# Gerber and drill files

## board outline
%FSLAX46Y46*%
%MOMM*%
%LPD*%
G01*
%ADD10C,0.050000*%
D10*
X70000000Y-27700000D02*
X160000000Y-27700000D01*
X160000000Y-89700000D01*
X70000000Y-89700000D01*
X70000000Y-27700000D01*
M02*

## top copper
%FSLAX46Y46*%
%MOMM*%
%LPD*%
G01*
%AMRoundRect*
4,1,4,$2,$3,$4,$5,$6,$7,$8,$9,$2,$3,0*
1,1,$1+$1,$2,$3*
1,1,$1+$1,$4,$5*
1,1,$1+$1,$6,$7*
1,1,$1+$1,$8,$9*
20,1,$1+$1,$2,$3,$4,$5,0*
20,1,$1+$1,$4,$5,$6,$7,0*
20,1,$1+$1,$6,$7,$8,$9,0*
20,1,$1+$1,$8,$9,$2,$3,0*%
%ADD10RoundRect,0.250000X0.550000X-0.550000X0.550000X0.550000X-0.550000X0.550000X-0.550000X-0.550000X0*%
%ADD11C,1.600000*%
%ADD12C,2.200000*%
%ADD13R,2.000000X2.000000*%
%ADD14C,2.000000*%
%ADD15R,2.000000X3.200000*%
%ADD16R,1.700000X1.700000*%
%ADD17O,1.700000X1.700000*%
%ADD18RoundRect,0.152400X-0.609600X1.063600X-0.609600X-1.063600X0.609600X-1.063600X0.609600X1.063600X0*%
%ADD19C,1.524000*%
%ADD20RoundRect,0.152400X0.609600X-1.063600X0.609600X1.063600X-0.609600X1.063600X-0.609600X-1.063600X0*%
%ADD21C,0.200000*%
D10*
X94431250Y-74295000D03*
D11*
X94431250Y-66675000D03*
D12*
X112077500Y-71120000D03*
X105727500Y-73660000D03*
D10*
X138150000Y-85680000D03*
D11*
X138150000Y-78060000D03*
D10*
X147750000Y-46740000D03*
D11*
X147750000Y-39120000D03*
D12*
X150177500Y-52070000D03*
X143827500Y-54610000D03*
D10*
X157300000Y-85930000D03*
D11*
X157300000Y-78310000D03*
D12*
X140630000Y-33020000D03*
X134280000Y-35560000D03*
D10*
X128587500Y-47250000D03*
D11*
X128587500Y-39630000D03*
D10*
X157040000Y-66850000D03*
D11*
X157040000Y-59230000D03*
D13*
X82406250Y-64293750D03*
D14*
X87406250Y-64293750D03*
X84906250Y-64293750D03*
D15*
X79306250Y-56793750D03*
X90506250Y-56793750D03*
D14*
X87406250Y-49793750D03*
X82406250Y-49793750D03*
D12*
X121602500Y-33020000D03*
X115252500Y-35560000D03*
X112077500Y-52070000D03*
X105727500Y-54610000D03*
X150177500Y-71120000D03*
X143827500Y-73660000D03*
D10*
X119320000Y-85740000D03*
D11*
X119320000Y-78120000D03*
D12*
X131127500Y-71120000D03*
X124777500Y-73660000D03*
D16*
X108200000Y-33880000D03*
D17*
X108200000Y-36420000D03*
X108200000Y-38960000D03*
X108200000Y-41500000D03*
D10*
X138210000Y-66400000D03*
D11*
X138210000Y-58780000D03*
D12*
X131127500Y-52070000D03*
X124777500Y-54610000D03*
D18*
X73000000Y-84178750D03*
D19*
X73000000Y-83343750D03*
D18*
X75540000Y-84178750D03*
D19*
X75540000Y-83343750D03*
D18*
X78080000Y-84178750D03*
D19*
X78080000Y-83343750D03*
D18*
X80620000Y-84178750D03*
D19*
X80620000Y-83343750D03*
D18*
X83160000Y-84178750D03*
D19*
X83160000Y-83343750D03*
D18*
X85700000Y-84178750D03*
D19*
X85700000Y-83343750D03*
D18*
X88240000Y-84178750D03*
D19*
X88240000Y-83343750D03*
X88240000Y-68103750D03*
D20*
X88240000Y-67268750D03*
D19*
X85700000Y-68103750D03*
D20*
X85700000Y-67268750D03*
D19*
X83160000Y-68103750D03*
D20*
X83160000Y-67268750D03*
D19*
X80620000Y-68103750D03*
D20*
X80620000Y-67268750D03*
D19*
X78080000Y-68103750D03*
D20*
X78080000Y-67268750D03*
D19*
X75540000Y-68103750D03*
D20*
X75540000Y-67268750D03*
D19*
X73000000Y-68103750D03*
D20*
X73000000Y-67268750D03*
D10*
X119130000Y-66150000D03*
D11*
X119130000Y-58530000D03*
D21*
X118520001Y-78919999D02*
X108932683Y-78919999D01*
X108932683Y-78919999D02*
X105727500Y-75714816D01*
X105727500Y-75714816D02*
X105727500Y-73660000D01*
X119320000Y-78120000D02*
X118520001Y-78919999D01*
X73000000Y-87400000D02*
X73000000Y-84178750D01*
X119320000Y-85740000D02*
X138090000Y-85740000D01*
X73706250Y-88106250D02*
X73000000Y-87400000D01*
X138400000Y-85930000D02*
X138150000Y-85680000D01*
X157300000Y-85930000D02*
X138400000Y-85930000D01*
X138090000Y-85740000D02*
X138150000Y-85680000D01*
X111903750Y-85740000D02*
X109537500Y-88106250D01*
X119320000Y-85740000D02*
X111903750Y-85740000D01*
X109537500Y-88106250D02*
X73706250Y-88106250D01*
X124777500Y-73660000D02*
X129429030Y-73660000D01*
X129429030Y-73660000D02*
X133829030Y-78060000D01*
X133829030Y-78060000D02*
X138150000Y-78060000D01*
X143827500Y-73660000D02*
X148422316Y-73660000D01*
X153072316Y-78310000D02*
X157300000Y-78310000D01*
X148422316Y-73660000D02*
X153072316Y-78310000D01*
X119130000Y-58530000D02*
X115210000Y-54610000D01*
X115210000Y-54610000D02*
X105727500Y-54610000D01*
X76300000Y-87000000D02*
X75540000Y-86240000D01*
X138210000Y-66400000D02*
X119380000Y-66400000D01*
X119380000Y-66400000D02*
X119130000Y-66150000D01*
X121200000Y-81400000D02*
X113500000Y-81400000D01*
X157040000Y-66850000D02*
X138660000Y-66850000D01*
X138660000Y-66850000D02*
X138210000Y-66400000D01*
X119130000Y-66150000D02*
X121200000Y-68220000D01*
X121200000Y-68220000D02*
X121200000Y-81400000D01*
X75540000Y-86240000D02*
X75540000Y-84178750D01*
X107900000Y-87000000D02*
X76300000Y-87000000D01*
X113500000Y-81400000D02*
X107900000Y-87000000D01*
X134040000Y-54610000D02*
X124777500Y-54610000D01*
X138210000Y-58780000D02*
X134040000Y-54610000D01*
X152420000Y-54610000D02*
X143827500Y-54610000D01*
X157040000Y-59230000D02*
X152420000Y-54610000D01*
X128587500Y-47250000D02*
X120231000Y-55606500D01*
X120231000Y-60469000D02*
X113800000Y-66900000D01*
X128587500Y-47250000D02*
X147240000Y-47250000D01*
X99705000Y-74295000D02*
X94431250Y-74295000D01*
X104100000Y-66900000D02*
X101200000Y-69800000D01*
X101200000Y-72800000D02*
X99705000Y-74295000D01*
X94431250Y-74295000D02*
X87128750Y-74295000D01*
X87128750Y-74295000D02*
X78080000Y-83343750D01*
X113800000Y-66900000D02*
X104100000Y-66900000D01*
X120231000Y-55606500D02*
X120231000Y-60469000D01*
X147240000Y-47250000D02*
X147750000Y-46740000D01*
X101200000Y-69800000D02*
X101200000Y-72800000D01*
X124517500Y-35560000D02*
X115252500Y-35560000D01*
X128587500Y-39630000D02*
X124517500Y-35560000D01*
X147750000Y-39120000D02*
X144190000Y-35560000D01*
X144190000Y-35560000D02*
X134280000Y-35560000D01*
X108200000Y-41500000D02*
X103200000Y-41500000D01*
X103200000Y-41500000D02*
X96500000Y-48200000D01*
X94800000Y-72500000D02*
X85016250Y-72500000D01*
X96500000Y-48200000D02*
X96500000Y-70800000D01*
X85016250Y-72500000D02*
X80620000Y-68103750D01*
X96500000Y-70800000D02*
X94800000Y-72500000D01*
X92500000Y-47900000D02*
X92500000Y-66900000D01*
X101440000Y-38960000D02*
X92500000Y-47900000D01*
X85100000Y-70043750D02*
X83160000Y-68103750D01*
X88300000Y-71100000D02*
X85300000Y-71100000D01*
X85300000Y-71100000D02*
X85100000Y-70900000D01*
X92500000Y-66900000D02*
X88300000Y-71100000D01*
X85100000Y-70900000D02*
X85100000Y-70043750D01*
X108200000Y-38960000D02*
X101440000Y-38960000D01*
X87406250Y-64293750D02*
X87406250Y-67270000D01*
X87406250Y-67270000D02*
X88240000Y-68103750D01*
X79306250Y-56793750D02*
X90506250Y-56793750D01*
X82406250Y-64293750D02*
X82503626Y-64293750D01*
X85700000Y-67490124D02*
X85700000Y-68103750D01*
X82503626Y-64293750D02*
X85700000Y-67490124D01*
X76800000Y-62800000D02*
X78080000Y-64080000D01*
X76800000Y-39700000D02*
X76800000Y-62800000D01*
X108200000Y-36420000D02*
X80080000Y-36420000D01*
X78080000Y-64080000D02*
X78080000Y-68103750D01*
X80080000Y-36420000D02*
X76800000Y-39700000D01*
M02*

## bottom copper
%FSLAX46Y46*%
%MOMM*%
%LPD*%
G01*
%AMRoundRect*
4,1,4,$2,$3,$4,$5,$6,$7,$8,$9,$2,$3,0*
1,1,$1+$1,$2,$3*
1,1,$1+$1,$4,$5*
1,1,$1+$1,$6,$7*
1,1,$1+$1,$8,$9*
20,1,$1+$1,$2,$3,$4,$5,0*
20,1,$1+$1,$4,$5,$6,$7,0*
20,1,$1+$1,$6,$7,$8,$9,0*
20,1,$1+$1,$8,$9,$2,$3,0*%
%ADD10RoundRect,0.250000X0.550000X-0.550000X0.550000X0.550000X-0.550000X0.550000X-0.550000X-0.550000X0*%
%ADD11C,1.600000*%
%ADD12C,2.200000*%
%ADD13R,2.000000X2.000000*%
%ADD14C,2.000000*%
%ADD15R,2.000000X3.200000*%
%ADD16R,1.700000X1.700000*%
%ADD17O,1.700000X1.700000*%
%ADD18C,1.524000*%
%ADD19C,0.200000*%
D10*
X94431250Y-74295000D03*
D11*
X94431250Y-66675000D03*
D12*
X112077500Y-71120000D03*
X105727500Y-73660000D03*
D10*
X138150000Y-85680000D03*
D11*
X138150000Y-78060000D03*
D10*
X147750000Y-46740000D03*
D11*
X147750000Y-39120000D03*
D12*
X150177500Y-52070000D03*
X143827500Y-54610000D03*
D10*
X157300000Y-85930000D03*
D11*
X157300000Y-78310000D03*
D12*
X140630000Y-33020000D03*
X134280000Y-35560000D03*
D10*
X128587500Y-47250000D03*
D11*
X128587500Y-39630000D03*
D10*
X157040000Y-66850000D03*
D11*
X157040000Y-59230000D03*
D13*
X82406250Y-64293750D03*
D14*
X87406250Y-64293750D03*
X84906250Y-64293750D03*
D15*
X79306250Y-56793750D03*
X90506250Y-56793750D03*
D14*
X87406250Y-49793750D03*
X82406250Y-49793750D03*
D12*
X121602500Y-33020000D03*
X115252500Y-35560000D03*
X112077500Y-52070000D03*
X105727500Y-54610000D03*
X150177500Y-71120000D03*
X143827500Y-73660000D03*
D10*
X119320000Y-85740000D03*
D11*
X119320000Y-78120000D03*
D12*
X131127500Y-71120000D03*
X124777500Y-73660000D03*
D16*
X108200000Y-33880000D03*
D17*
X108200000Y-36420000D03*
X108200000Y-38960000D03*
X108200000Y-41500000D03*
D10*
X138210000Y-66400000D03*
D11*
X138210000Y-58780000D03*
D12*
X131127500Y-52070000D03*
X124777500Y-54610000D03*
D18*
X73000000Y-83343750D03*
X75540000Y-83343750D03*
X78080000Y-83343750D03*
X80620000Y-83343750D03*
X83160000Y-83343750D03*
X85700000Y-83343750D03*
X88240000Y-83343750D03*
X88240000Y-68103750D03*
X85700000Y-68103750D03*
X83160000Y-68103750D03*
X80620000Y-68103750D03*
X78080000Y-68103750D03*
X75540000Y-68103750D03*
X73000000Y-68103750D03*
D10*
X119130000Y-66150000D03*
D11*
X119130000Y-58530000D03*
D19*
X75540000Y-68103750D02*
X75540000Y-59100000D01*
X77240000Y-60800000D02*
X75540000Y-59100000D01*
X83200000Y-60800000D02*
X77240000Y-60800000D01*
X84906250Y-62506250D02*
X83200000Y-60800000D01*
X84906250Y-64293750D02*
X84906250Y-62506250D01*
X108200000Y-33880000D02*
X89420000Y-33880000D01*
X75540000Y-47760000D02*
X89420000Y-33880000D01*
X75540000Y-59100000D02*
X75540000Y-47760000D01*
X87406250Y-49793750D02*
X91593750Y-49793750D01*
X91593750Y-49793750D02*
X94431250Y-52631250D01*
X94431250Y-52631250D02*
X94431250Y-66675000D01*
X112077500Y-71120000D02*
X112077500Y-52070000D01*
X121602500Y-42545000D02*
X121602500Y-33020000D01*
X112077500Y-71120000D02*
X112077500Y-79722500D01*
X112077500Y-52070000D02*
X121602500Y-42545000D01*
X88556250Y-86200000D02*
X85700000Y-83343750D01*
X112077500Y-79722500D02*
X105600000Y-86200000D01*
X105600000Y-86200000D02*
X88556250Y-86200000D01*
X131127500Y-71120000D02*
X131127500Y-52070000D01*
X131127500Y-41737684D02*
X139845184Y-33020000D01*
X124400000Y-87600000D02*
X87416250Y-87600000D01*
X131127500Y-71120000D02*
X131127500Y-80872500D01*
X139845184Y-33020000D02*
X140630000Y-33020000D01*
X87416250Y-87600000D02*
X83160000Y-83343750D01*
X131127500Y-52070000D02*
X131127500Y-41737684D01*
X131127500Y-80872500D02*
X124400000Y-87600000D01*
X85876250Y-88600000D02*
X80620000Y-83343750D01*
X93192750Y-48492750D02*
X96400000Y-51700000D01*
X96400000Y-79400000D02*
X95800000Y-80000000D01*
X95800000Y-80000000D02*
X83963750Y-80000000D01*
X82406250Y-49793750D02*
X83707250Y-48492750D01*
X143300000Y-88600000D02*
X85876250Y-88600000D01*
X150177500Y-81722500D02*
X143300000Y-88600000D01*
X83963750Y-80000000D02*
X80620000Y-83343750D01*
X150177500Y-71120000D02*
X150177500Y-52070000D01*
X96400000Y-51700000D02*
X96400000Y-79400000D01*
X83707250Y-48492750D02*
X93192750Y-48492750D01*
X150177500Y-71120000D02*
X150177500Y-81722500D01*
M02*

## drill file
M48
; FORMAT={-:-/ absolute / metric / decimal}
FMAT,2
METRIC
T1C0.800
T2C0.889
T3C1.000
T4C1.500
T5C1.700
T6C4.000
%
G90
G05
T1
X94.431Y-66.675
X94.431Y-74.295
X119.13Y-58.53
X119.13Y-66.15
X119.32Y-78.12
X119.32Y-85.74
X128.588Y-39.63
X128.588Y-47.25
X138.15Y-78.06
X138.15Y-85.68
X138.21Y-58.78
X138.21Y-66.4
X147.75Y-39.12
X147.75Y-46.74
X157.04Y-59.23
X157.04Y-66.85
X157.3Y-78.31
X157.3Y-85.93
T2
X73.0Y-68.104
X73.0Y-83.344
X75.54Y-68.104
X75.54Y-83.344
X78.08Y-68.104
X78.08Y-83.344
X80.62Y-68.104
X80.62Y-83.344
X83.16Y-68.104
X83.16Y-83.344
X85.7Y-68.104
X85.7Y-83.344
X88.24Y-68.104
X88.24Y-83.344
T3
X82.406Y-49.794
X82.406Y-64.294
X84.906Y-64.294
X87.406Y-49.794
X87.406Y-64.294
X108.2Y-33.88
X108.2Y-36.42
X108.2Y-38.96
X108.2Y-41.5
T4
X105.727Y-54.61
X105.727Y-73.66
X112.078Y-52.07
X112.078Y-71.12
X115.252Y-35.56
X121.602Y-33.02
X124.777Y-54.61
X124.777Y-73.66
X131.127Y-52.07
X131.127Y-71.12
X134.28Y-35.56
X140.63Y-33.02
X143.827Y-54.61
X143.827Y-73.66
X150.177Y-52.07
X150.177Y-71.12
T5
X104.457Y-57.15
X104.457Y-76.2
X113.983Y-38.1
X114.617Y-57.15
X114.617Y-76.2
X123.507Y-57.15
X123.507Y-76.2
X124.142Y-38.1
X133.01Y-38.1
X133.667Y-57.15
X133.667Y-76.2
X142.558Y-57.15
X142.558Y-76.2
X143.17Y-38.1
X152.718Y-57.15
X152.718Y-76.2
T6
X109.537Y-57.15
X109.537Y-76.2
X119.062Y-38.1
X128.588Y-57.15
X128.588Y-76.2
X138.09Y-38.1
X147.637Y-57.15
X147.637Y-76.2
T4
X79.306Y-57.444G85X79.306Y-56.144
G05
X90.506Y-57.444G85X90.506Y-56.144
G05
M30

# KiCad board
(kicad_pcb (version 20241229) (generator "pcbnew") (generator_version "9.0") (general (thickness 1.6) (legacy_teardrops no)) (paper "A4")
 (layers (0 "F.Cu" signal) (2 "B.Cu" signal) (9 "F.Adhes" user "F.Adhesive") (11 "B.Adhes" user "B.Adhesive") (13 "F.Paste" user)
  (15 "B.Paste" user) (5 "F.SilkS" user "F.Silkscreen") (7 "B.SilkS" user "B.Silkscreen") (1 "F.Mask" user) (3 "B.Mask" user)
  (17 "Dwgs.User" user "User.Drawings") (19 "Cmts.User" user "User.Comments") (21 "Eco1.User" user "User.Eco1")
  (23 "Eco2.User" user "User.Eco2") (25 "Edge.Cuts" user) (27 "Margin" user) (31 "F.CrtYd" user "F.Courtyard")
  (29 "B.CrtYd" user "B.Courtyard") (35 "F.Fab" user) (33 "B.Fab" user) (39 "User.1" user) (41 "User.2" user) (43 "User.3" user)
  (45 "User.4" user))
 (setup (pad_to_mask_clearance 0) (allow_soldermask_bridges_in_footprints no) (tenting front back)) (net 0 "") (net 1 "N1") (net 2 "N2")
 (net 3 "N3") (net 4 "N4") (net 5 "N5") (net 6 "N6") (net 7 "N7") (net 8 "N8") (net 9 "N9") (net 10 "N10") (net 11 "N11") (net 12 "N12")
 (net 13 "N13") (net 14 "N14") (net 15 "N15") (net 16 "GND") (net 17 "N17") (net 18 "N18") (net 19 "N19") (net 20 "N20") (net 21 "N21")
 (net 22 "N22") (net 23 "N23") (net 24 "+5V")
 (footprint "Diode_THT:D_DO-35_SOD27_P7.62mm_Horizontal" (layer "F.Cu") (at 94.43125 74.295 90)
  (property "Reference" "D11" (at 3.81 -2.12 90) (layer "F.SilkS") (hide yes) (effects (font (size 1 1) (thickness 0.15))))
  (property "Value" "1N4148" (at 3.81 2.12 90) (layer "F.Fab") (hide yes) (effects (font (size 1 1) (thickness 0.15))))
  (pad "1" thru_hole roundrect (at 0 0 90) (size 1.6 1.6) (drill 0.8) (layers "*.Cu" "*.Mask") (remove_unused_layers no)
   (roundrect_rratio 0.15625) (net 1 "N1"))
  (pad "2" thru_hole circle (at 7.62 0 90) (size 1.6 1.6) (drill 0.8) (layers "*.Cu" "*.Mask") (remove_unused_layers no) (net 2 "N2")))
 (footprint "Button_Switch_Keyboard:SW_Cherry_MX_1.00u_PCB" (layer "F.Cu") (at 112.0775 71.12)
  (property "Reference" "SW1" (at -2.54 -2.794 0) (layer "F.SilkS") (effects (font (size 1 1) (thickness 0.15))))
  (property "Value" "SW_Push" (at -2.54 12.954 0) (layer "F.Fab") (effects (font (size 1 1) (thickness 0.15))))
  (pad "" np_thru_hole circle (at -7.62 5.08) (size 1.7 1.7) (drill 1.7) (layers "*.Cu" "*.Mask"))
  (pad "" np_thru_hole circle (at -2.54 5.08) (size 4 4) (drill 4) (layers "*.Cu" "*.Mask"))
  (pad "" np_thru_hole circle (at 2.54 5.08) (size 1.7 1.7) (drill 1.7) (layers "*.Cu" "*.Mask"))
  (pad "1" thru_hole circle (at 0 0) (size 2.2 2.2) (drill 1.5) (layers "*.Cu" "*.Mask") (remove_unused_layers no) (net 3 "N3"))
  (pad "2" thru_hole circle (at -6.35 2.54) (size 2.2 2.2) (drill 1.5) (layers "*.Cu" "*.Mask") (remove_unused_layers no) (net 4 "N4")))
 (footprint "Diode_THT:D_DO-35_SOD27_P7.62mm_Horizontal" (layer "F.Cu") (at 138.15 85.68 90)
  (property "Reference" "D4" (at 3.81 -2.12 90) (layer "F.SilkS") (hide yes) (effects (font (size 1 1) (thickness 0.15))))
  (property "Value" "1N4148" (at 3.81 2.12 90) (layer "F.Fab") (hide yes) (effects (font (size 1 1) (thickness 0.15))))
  (pad "1" thru_hole roundrect (at 0 0 90) (size 1.6 1.6) (drill 0.8) (layers "*.Cu" "*.Mask") (remove_unused_layers no)
   (roundrect_rratio 0.15625) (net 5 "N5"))
  (pad "2" thru_hole circle (at 7.62 0 90) (size 1.6 1.6) (drill 0.8) (layers "*.Cu" "*.Mask") (remove_unused_layers no) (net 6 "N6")))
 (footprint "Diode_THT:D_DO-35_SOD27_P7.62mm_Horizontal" (layer "F.Cu") (at 147.75 46.74 90)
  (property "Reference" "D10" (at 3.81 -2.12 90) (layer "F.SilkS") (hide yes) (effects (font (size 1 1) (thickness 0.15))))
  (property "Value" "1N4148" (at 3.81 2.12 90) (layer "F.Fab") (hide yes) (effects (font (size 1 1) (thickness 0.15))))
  (pad "1" thru_hole roundrect (at 0 0 90) (size 1.6 1.6) (drill 0.8) (layers "*.Cu" "*.Mask") (remove_unused_layers no)
   (roundrect_rratio 0.15625) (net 1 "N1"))
  (pad "2" thru_hole circle (at 7.62 0 90) (size 1.6 1.6) (drill 0.8) (layers "*.Cu" "*.Mask") (remove_unused_layers no) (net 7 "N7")))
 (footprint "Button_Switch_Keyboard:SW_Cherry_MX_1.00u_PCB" (layer "F.Cu") (at 150.1775 52.07)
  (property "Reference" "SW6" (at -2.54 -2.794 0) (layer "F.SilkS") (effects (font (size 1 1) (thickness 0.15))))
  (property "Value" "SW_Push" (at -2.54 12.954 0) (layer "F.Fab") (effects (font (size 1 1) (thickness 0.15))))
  (pad "" np_thru_hole circle (at -7.62 5.08) (size 1.7 1.7) (drill 1.7) (layers "*.Cu" "*.Mask"))
  (pad "" np_thru_hole circle (at -2.54 5.08) (size 4 4) (drill 4) (layers "*.Cu" "*.Mask"))
  (pad "" np_thru_hole circle (at 2.54 5.08) (size 1.7 1.7) (drill 1.7) (layers "*.Cu" "*.Mask"))
  (pad "1" thru_hole circle (at 0 0) (size 2.2 2.2) (drill 1.5) (layers "*.Cu" "*.Mask") (remove_unused_layers no) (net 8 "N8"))
  (pad "2" thru_hole circle (at -6.35 2.54) (size 2.2 2.2) (drill 1.5) (layers "*.Cu" "*.Mask") (remove_unused_layers no) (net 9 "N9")))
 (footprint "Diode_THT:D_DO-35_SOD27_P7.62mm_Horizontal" (layer "F.Cu") (at 157.3 85.93 90)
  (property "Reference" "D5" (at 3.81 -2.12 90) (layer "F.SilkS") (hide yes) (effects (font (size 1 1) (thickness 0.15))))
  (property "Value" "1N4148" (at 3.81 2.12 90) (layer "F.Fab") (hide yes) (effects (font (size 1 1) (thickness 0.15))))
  (pad "1" thru_hole roundrect (at 0 0 90) (size 1.6 1.6) (drill 0.8) (layers "*.Cu" "*.Mask") (remove_unused_layers no)
   (roundrect_rratio 0.15625) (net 5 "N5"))
  (pad "2" thru_hole circle (at 7.62 0 90) (size 1.6 1.6) (drill 0.8) (layers "*.Cu" "*.Mask") (remove_unused_layers no) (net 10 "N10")))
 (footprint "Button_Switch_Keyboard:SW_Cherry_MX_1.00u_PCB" (layer "F.Cu") (at 140.63 33.02)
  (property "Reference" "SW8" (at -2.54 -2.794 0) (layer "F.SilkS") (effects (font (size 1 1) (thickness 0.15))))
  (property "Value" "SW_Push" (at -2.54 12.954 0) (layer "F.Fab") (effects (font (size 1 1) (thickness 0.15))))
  (pad "" np_thru_hole circle (at -7.62 5.08) (size 1.7 1.7) (drill 1.7) (layers "*.Cu" "*.Mask"))
  (pad "" np_thru_hole circle (at -2.54 5.08) (size 4 4) (drill 4) (layers "*.Cu" "*.Mask"))
  (pad "" np_thru_hole circle (at 2.54 5.08) (size 1.7 1.7) (drill 1.7) (layers "*.Cu" "*.Mask"))
  (pad "1" thru_hole circle (at 0 0) (size 2.2 2.2) (drill 1.5) (layers "*.Cu" "*.Mask") (remove_unused_layers no) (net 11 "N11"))
  (pad "2" thru_hole circle (at -6.35 2.54) (size 2.2 2.2) (drill 1.5) (layers "*.Cu" "*.Mask") (remove_unused_layers no) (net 7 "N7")))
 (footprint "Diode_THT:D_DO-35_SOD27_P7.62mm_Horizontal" (layer "F.Cu") (at 128.5875 47.25 90)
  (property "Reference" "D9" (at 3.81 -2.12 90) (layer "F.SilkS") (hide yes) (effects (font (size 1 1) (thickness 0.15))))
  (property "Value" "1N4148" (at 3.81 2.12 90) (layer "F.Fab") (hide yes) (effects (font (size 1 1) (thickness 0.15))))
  (pad "1" thru_hole roundrect (at 0 0 90) (size 1.6 1.6) (drill 0.8) (layers "*.Cu" "*.Mask") (remove_unused_layers no)
   (roundrect_rratio 0.15625) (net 1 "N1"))
  (pad "2" thru_hole circle (at 7.62 0 90) (size 1.6 1.6) (drill 0.8) (layers "*.Cu" "*.Mask") (remove_unused_layers no) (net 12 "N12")))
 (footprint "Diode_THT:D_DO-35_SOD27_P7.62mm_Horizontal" (layer "F.Cu") (at 157.04 66.85 90)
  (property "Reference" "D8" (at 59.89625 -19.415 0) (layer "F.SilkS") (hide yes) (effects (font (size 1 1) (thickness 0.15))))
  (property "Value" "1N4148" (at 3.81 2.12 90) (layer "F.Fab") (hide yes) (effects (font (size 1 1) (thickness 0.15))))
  (pad "1" thru_hole roundrect (at 0 0 90) (size 1.6 1.6) (drill 0.8) (layers "*.Cu" "*.Mask") (remove_unused_layers no)
   (roundrect_rratio 0.15625) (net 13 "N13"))
  (pad "2" thru_hole circle (at 7.62 0 90) (size 1.6 1.6) (drill 0.8) (layers "*.Cu" "*.Mask") (remove_unused_layers no) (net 9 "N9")))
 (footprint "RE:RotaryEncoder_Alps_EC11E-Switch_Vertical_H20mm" (layer "F.Cu") (at 82.40625 64.29375 90)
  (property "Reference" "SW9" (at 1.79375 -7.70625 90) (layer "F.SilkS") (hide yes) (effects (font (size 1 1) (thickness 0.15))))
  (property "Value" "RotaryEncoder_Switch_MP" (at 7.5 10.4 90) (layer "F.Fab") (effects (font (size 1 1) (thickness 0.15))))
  (pad "A" thru_hole rect (at 0 0 90) (size 2 2) (drill 1) (layers "*.Cu" "*.Mask") (remove_unused_layers no) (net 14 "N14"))
  (pad "B" thru_hole circle (at 0 5 90) (size 2 2) (drill 1) (layers "*.Cu" "*.Mask") (remove_unused_layers no) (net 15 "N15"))
  (pad "C" thru_hole circle (at 0 2.5 90) (size 2 2) (drill 1) (layers "*.Cu" "*.Mask") (remove_unused_layers no) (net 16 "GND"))
  (pad "MP" thru_hole rect (at 7.5 -3.1 90) (size 3.2 2) (drill oval 2.8 1.5) (layers "*.Cu" "*.Mask") (remove_unused_layers no)
   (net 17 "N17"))
  (pad "MP" thru_hole rect (at 7.5 8.1 90) (size 3.2 2) (drill oval 2.8 1.5) (layers "*.Cu" "*.Mask") (remove_unused_layers no)
   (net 17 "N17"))
  (pad "S1" thru_hole circle (at 14.5 5 90) (size 2 2) (drill 1) (layers "*.Cu" "*.Mask") (remove_unused_layers no) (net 2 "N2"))
  (pad "S2" thru_hole circle (at 14.5 0 90) (size 2 2) (drill 1) (layers "*.Cu" "*.Mask") (remove_unused_layers no) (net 8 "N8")))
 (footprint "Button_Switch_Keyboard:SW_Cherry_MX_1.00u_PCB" (layer "F.Cu") (at 121.6025 33.02)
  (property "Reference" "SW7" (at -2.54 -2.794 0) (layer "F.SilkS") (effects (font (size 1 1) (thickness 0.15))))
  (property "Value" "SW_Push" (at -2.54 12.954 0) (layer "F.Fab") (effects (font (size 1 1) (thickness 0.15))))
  (pad "" np_thru_hole circle (at -7.62 5.08) (size 1.7 1.7) (drill 1.7) (layers "*.Cu" "*.Mask"))
  (pad "" np_thru_hole circle (at -2.54 5.08) (size 4 4) (drill 4) (layers "*.Cu" "*.Mask"))
  (pad "" np_thru_hole circle (at 2.54 5.08) (size 1.7 1.7) (drill 1.7) (layers "*.Cu" "*.Mask"))
  (pad "1" thru_hole circle (at 0 0) (size 2.2 2.2) (drill 1.5) (layers "*.Cu" "*.Mask") (remove_unused_layers no) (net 3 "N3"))
  (pad "2" thru_hole circle (at -6.35 2.54) (size 2.2 2.2) (drill 1.5) (layers "*.Cu" "*.Mask") (remove_unused_layers no) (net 12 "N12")))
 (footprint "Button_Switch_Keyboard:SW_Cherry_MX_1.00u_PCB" (layer "F.Cu") (at 112.0775 52.07)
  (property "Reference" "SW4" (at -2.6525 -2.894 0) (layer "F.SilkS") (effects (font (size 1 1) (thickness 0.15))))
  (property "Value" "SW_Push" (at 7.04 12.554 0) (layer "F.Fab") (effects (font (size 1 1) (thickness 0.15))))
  (pad "" np_thru_hole circle (at -7.62 5.08) (size 1.7 1.7) (drill 1.7) (layers "*.Cu" "*.Mask"))
  (pad "" np_thru_hole circle (at -2.54 5.08) (size 4 4) (drill 4) (layers "*.Cu" "*.Mask"))
  (pad "" np_thru_hole circle (at 2.54 5.08) (size 1.7 1.7) (drill 1.7) (layers "*.Cu" "*.Mask"))
  (pad "1" thru_hole circle (at 0 0) (size 2.2 2.2) (drill 1.5) (layers "*.Cu" "*.Mask") (remove_unused_layers no) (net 3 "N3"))
  (pad "2" thru_hole circle (at -6.35 2.54) (size 2.2 2.2) (drill 1.5) (layers "*.Cu" "*.Mask") (remove_unused_layers no) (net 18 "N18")))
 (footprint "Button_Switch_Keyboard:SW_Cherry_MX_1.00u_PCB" (layer "F.Cu") (at 150.1775 71.12)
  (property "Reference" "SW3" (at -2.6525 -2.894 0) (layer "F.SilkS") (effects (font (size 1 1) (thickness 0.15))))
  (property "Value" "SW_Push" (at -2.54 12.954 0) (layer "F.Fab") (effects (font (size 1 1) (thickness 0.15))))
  (pad "" np_thru_hole circle (at -7.62 5.08) (size 1.7 1.7) (drill 1.7) (layers "*.Cu" "*.Mask"))
  (pad "" np_thru_hole circle (at -2.54 5.08) (size 4 4) (drill 4) (layers "*.Cu" "*.Mask"))
  (pad "" np_thru_hole circle (at 2.54 5.08) (size 1.7 1.7) (drill 1.7) (layers "*.Cu" "*.Mask"))
  (pad "1" thru_hole circle (at 0 0) (size 2.2 2.2) (drill 1.5) (layers "*.Cu" "*.Mask") (remove_unused_layers no) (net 8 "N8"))
  (pad "2" thru_hole circle (at -6.35 2.54) (size 2.2 2.2) (drill 1.5) (layers "*.Cu" "*.Mask") (remove_unused_layers no) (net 10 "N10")))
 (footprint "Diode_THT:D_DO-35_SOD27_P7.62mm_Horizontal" (layer "F.Cu") (at 119.32 85.74 90)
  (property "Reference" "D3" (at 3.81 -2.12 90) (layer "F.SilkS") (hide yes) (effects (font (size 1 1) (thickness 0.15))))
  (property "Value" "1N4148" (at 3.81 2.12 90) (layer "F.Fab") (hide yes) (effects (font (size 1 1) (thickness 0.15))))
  (pad "1" thru_hole roundrect (at 0 0 90) (size 1.6 1.6) (drill 0.8) (layers "*.Cu" "*.Mask") (remove_unused_layers no)
   (roundrect_rratio 0.15625) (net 5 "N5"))
  (pad "2" thru_hole circle (at 7.62 0 90) (size 1.6 1.6) (drill 0.8) (layers "*.Cu" "*.Mask") (remove_unused_layers no) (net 4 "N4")))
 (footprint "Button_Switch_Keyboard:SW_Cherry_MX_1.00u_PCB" (layer "F.Cu") (at 131.1275 71.12)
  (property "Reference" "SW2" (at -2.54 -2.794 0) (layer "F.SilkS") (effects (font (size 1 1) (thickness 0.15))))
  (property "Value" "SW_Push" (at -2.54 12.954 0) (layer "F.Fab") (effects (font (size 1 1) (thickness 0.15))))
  (pad "" np_thru_hole circle (at -7.62 5.08) (size 1.7 1.7) (drill 1.7) (layers "*.Cu" "*.Mask"))
  (pad "" np_thru_hole circle (at -2.54 5.08) (size 4 4) (drill 4) (layers "*.Cu" "*.Mask"))
  (pad "" np_thru_hole circle (at 2.54 5.08) (size 1.7 1.7) (drill 1.7) (layers "*.Cu" "*.Mask"))
  (pad "1" thru_hole circle (at 0 0) (size 2.2 2.2) (drill 1.5) (layers "*.Cu" "*.Mask") (remove_unused_layers no) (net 11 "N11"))
  (pad "2" thru_hole circle (at -6.35 2.54) (size 2.2 2.2) (drill 1.5) (layers "*.Cu" "*.Mask") (remove_unused_layers no) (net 6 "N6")))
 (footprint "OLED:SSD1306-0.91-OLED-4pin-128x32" (layer "F.Cu") (at 71.7 31.69)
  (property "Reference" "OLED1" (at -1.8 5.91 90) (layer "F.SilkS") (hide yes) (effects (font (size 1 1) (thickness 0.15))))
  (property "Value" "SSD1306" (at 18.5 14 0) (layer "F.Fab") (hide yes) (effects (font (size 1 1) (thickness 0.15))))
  (pad "1" thru_hole rect (at 36.5 2.19) (size 1.7 1.7) (drill 1) (layers "*.Cu" "*.Mask") (remove_unused_layers no) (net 16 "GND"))
  (pad "2" thru_hole oval (at 36.5 4.73) (size 1.7 1.7) (drill 1) (layers "*.Cu" "*.Mask") (remove_unused_layers no) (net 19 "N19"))
  (pad "3" thru_hole oval (at 36.5 7.27) (size 1.7 1.7) (drill 1) (layers "*.Cu" "*.Mask") (remove_unused_layers no) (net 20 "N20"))
  (pad "4" thru_hole oval (at 36.5 9.81) (size 1.7 1.7) (drill 1) (layers "*.Cu" "*.Mask") (remove_unused_layers no) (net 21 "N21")))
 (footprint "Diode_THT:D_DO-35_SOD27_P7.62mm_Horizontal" (layer "F.Cu") (at 138.21 66.4 90)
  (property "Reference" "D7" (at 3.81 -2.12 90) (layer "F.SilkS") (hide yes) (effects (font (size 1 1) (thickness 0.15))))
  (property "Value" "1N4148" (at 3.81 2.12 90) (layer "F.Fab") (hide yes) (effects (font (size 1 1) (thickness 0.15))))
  (pad "1" thru_hole roundrect (at 0 0 90) (size 1.6 1.6) (drill 0.8) (layers "*.Cu" "*.Mask") (remove_unused_layers no)
   (roundrect_rratio 0.15625) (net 13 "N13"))
  (pad "2" thru_hole circle (at 7.62 0 90) (size 1.6 1.6) (drill 0.8) (layers "*.Cu" "*.Mask") (remove_unused_layers no) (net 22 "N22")))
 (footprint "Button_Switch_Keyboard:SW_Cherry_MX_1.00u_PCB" (layer "F.Cu") (at 131.1275 52.07)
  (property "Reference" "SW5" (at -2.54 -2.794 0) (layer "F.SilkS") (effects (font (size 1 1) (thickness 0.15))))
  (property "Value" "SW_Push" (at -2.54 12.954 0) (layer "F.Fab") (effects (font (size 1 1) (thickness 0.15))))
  (pad "" np_thru_hole circle (at -7.62 5.08) (size 1.7 1.7) (drill 1.7) (layers "*.Cu" "*.Mask"))
  (pad "" np_thru_hole circle (at -2.54 5.08) (size 4 4) (drill 4) (layers "*.Cu" "*.Mask"))
  (pad "" np_thru_hole circle (at 2.54 5.08) (size 1.7 1.7) (drill 1.7) (layers "*.Cu" "*.Mask"))
  (pad "1" thru_hole circle (at 0 0) (size 2.2 2.2) (drill 1.5) (layers "*.Cu" "*.Mask") (remove_unused_layers no) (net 11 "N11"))
  (pad "2" thru_hole circle (at -6.35 2.54) (size 2.2 2.2) (drill 1.5) (layers "*.Cu" "*.Mask") (remove_unused_layers no) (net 22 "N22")))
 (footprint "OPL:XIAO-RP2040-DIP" (layer "F.Cu") (at 80.62 75.72375 90)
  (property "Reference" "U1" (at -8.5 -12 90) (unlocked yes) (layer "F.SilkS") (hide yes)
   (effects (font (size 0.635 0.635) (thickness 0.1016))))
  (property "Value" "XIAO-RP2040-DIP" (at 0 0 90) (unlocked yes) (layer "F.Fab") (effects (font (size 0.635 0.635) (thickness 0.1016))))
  (pad "1" smd roundrect (at -8.455 -7.62 270) (size 2.432 1.524) (layers "F.Cu" "F.Mask") (roundrect_rratio 0.1) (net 5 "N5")
   (thermal_bridge_angle 45))
  (pad "1" thru_hole circle (at -7.62 -7.62 270) (size 1.524 1.524) (drill 0.889) (layers "*.Cu" "*.Mask") (remove_unused_layers no)
   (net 5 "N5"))
  (pad "2" smd roundrect (at -8.455 -5.08 270) (size 2.432 1.524) (layers "F.Cu" "F.Mask") (roundrect_rratio 0.1) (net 13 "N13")
   (thermal_bridge_angle 45))
  (pad "2" thru_hole circle (at -7.62 -5.08 270) (size 1.524 1.524) (drill 0.889) (layers "*.Cu" "*.Mask") (remove_unused_layers no)
   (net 13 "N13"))
  (pad "3" smd roundrect (at -8.455 -2.54 270) (size 2.432 1.524) (layers "F.Cu" "F.Mask") (roundrect_rratio 0.1) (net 1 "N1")
   (thermal_bridge_angle 45))
  (pad "3" thru_hole circle (at -7.62 -2.54 270) (size 1.524 1.524) (drill 0.889) (layers "*.Cu" "*.Mask") (remove_unused_layers no)
   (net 1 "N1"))
  (pad "4" smd roundrect (at -8.455 0 270) (size 2.432 1.524) (layers "F.Cu" "F.Mask") (roundrect_rratio 0.1) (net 8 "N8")
   (thermal_bridge_angle 45))
  (pad "4" thru_hole circle (at -7.62 0 270) (size 1.524 1.524) (drill 0.889) (layers "*.Cu" "*.Mask") (remove_unused_layers no)
   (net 8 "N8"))
  (pad "5" smd roundrect (at -8.455 2.54 270) (size 2.432 1.524) (layers "F.Cu" "F.Mask") (roundrect_rratio 0.1) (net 11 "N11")
   (thermal_bridge_angle 45))
  (pad "5" thru_hole circle (at -7.62 2.54 270) (size 1.524 1.524) (drill 0.889) (layers "*.Cu" "*.Mask") (remove_unused_layers no)
   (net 11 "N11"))
  (pad "6" smd roundrect (at -8.455 5.08 270) (size 2.432 1.524) (layers "F.Cu" "F.Mask") (roundrect_rratio 0.1) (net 3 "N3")
   (thermal_bridge_angle 45))
  (pad "6" thru_hole circle (at -7.62 5.08 270) (size 1.524 1.524) (drill 0.889) (layers "*.Cu" "*.Mask") (remove_unused_layers no)
   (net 3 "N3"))
  (pad "7" smd roundrect (at -8.455 7.62 270) (size 2.432 1.524) (layers "F.Cu" "F.Mask") (roundrect_rratio 0.1) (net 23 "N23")
   (thermal_bridge_angle 45))
  (pad "7" thru_hole circle (at -7.62 7.62 270) (size 1.524 1.524) (drill 0.889) (layers "*.Cu" "*.Mask") (remove_unused_layers no)
   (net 23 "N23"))
  (pad "8" thru_hole circle (at 7.62 7.62 90) (size 1.524 1.524) (drill 0.889) (layers "*.Cu" "*.Mask") (remove_unused_layers no)
   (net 15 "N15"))
  (pad "8" smd roundrect (at 8.455 7.62 90) (size 2.432 1.524) (layers "F.Cu" "F.Mask") (roundrect_rratio 0.1) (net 15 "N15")
   (thermal_bridge_angle 45))
  (pad "9" thru_hole circle (at 7.62 5.08 90) (size 1.524 1.524) (drill 0.889) (layers "*.Cu" "*.Mask") (remove_unused_layers no)
   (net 14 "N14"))
  (pad "9" smd roundrect (at 8.455 5.08 90) (size 2.432 1.524) (layers "F.Cu" "F.Mask") (roundrect_rratio 0.1) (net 14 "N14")
   (thermal_bridge_angle 45))
  (pad "10" thru_hole circle (at 7.62 2.54 90) (size 1.524 1.524) (drill 0.889) (layers "*.Cu" "*.Mask") (remove_unused_layers no)
   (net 20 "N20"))
  (pad "10" smd roundrect (at 8.455 2.54 90) (size 2.432 1.524) (layers "F.Cu" "F.Mask") (roundrect_rratio 0.1) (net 20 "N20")
   (thermal_bridge_angle 45))
  (pad "11" thru_hole circle (at 7.62 0 90) (size 1.524 1.524) (drill 0.889) (layers "*.Cu" "*.Mask") (remove_unused_layers no)
   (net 21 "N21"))
  (pad "11" smd roundrect (at 8.455 0 90) (size 2.432 1.524) (layers "F.Cu" "F.Mask") (roundrect_rratio 0.1) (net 21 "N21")
   (thermal_bridge_angle 45))
  (pad "12" thru_hole circle (at 7.62 -2.54 90) (size 1.524 1.524) (drill 0.889) (layers "*.Cu" "*.Mask") (remove_unused_layers no)
   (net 19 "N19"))
  (pad "12" smd roundrect (at 8.455 -2.54 90) (size 2.432 1.524) (layers "F.Cu" "F.Mask") (roundrect_rratio 0.1) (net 19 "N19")
   (thermal_bridge_angle 45))
  (pad "13" thru_hole circle (at 7.62 -5.08 90) (size 1.524 1.524) (drill 0.889) (layers "*.Cu" "*.Mask") (remove_unused_layers no)
   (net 16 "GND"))
  (pad "13" smd roundrect (at 8.455 -5.08 90) (size 2.432 1.524) (layers "F.Cu" "F.Mask") (roundrect_rratio 0.1) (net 16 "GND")
   (thermal_bridge_angle 45))
  (pad "14" thru_hole circle (at 7.62 -7.62 90) (size 1.524 1.524) (drill 0.889) (layers "*.Cu" "*.Mask") (remove_unused_layers no)
   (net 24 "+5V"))
  (pad "14" smd roundrect (at 8.455 -7.62 90) (size 2.432 1.524) (layers "F.Cu" "F.Mask") (roundrect_rratio 0.1) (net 24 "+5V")
   (thermal_bridge_angle 45)))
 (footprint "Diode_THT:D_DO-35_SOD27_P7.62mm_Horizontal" (layer "F.Cu") (at 119.13 66.15 90)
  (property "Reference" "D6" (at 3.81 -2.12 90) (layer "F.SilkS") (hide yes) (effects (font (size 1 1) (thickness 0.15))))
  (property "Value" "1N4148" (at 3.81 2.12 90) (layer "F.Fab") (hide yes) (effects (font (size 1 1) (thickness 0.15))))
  (pad "1" thru_hole roundrect (at 0 0 90) (size 1.6 1.6) (drill 0.8) (layers "*.Cu" "*.Mask") (remove_unused_layers no)
   (roundrect_rratio 0.15625) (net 13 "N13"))
  (pad "2" thru_hole circle (at 7.62 0 90) (size 1.6 1.6) (drill 0.8) (layers "*.Cu" "*.Mask") (remove_unused_layers no) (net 18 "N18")))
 (gr_rect (start 70 27.7) (end 160 89.7) (stroke (width 0.05) (type default)) (fill no) (layer "Edge.Cuts"))
 (segment (start 75.54 68.10375) (end 75.54 59.1) (width 0.2) (layer "B.Cu") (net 16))
 (segment (start 77.24 60.8) (end 75.54 59.1) (width 0.2) (layer "B.Cu") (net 16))
 (segment (start 83.2 60.8) (end 77.24 60.8) (width 0.2) (layer "B.Cu") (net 16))
 (segment (start 84.90625 62.50625) (end 83.2 60.8) (width 0.2) (layer "B.Cu") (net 16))
 (segment (start 84.90625 64.29375) (end 84.90625 62.50625) (width 0.2) (layer "B.Cu") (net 16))
 (segment (start 108.2 33.88) (end 89.42 33.88) (width 0.2) (layer "B.Cu") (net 16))
 (segment (start 75.54 47.76) (end 89.42 33.88) (width 0.2) (layer "B.Cu") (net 16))
 (segment (start 75.54 59.1) (end 75.54 47.76) (width 0.2) (layer "B.Cu") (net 16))
 (segment (start 118.520001 78.919999) (end 108.932683 78.919999) (width 0.2) (layer "F.Cu") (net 4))
 (segment (start 108.932683 78.919999) (end 105.7275 75.714816) (width 0.2) (layer "F.Cu") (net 4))
 (segment (start 105.7275 75.714816) (end 105.7275 73.66) (width 0.2) (layer "F.Cu") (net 4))
 (segment (start 119.32 78.12) (end 118.520001 78.919999) (width 0.2) (layer "F.Cu") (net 4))
 (segment (start 73 87.4) (end 73 84.17875) (width 0.2) (layer "F.Cu") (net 5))
 (segment (start 119.32 85.74) (end 138.09 85.74) (width 0.2) (layer "F.Cu") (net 5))
 (segment (start 73.70625 88.10625) (end 73 87.4) (width 0.2) (layer "F.Cu") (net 5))
 (segment (start 138.4 85.93) (end 138.15 85.68) (width 0.2) (layer "F.Cu") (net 5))
 (segment (start 157.3 85.93) (end 138.4 85.93) (width 0.2) (layer "F.Cu") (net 5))
 (segment (start 138.09 85.74) (end 138.15 85.68) (width 0.2) (layer "F.Cu") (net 5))
 (segment (start 111.90375 85.74) (end 109.5375 88.10625) (width 0.2) (layer "F.Cu") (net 5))
 (segment (start 119.32 85.74) (end 111.90375 85.74) (width 0.2) (layer "F.Cu") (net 5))
 (segment (start 109.5375 88.10625) (end 73.70625 88.10625) (width 0.2) (layer "F.Cu") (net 5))
 (segment (start 124.7775 73.66) (end 129.42903 73.66) (width 0.2) (layer "F.Cu") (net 6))
 (segment (start 129.42903 73.66) (end 133.82903 78.06) (width 0.2) (layer "F.Cu") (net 6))
 (segment (start 133.82903 78.06) (end 138.15 78.06) (width 0.2) (layer "F.Cu") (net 6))
 (segment (start 143.8275 73.66) (end 148.422316 73.66) (width 0.2) (layer "F.Cu") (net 10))
 (segment (start 153.072316 78.31) (end 157.3 78.31) (width 0.2) (layer "F.Cu") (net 10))
 (segment (start 148.422316 73.66) (end 153.072316 78.31) (width 0.2) (layer "F.Cu") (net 10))
 (segment (start 119.13 58.53) (end 115.21 54.61) (width 0.2) (layer "F.Cu") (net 18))
 (segment (start 115.21 54.61) (end 105.7275 54.61) (width 0.2) (layer "F.Cu") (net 18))
 (segment (start 76.3 87) (end 75.54 86.24) (width 0.2) (layer "F.Cu") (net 13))
 (segment (start 138.21 66.4) (end 119.38 66.4) (width 0.2) (layer "F.Cu") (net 13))
 (segment (start 119.38 66.4) (end 119.13 66.15) (width 0.2) (layer "F.Cu") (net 13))
 (segment (start 121.2 81.4) (end 113.5 81.4) (width 0.2) (layer "F.Cu") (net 13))
 (segment (start 157.04 66.85) (end 138.66 66.85) (width 0.2) (layer "F.Cu") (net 13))
 (segment (start 138.66 66.85) (end 138.21 66.4) (width 0.2) (layer "F.Cu") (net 13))
 (segment (start 119.13 66.15) (end 121.2 68.22) (width 0.2) (layer "F.Cu") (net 13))
 (segment (start 121.2 68.22) (end 121.2 81.4) (width 0.2) (layer "F.Cu") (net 13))
 (segment (start 75.54 86.24) (end 75.54 84.17875) (width 0.2) (layer "F.Cu") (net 13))
 (segment (start 107.9 87) (end 76.3 87) (width 0.2) (layer "F.Cu") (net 13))
 (segment (start 113.5 81.4) (end 107.9 87) (width 0.2) (layer "F.Cu") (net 13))
 (segment (start 134.04 54.61) (end 124.7775 54.61) (width 0.2) (layer "F.Cu") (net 22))
 (segment (start 138.21 58.78) (end 134.04 54.61) (width 0.2) (layer "F.Cu") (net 22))
 (segment (start 152.42 54.61) (end 143.8275 54.61) (width 0.2) (layer "F.Cu") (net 9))
 (segment (start 157.04 59.23) (end 152.42 54.61) (width 0.2) (layer "F.Cu") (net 9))
 (segment (start 128.5875 47.25) (end 120.231 55.6065) (width 0.2) (layer "F.Cu") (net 1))
 (segment (start 120.231 60.469) (end 113.8 66.9) (width 0.2) (layer "F.Cu") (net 1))
 (segment (start 128.5875 47.25) (end 147.24 47.25) (width 0.2) (layer "F.Cu") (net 1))
 (segment (start 99.705 74.295) (end 94.43125 74.295) (width 0.2) (layer "F.Cu") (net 1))
 (segment (start 104.1 66.9) (end 101.2 69.8) (width 0.2) (layer "F.Cu") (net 1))
 (segment (start 101.2 72.8) (end 99.705 74.295) (width 0.2) (layer "F.Cu") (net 1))
 (segment (start 94.43125 74.295) (end 87.12875 74.295) (width 0.2) (layer "F.Cu") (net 1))
 (segment (start 87.12875 74.295) (end 78.08 83.34375) (width 0.2) (layer "F.Cu") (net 1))
 (segment (start 113.8 66.9) (end 104.1 66.9) (width 0.2) (layer "F.Cu") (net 1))
 (segment (start 120.231 55.6065) (end 120.231 60.469) (width 0.2) (layer "F.Cu") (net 1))
 (segment (start 147.24 47.25) (end 147.75 46.74) (width 0.2) (layer "F.Cu") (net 1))
 (segment (start 101.2 69.8) (end 101.2 72.8) (width 0.2) (layer "F.Cu") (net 1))
 (segment (start 124.5175 35.56) (end 115.2525 35.56) (width 0.2) (layer "F.Cu") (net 12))
 (segment (start 128.5875 39.63) (end 124.5175 35.56) (width 0.2) (layer "F.Cu") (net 12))
 (segment (start 147.75 39.12) (end 144.19 35.56) (width 0.2) (layer "F.Cu") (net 7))
 (segment (start 144.19 35.56) (end 134.28 35.56) (width 0.2) (layer "F.Cu") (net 7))
 (segment (start 87.40625 49.79375) (end 91.59375 49.79375) (width 0.2) (layer "B.Cu") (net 2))
 (segment (start 91.59375 49.79375) (end 94.43125 52.63125) (width 0.2) (layer "B.Cu") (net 2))
 (segment (start 94.43125 52.63125) (end 94.43125 66.675) (width 0.2) (layer "B.Cu") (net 2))
 (segment (start 108.2 41.5) (end 103.2 41.5) (width 0.2) (layer "F.Cu") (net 21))
 (segment (start 103.2 41.5) (end 96.5 48.2) (width 0.2) (layer "F.Cu") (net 21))
 (segment (start 94.8 72.5) (end 85.01625 72.5) (width 0.2) (layer "F.Cu") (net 21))
 (segment (start 96.5 48.2) (end 96.5 70.8) (width 0.2) (layer "F.Cu") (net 21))
 (segment (start 85.01625 72.5) (end 80.62 68.10375) (width 0.2) (layer "F.Cu") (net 21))
 (segment (start 96.5 70.8) (end 94.8 72.5) (width 0.2) (layer "F.Cu") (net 21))
 (segment (start 92.5 47.9) (end 92.5 66.9) (width 0.2) (layer "F.Cu") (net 20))
 (segment (start 101.44 38.96) (end 92.5 47.9) (width 0.2) (layer "F.Cu") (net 20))
 (segment (start 85.1 70.04375) (end 83.16 68.10375) (width 0.2) (layer "F.Cu") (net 20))
 (segment (start 88.3 71.1) (end 85.3 71.1) (width 0.2) (layer "F.Cu") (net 20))
 (segment (start 85.3 71.1) (end 85.1 70.9) (width 0.2) (layer "F.Cu") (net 20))
 (segment (start 92.5 66.9) (end 88.3 71.1) (width 0.2) (layer "F.Cu") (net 20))
 (segment (start 85.1 70.9) (end 85.1 70.04375) (width 0.2) (layer "F.Cu") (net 20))
 (segment (start 108.2 38.96) (end 101.44 38.96) (width 0.2) (layer "F.Cu") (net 20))
 (segment (start 112.0775 71.12) (end 112.0775 52.07) (width 0.2) (layer "B.Cu") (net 3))
 (segment (start 121.6025 42.545) (end 121.6025 33.02) (width 0.2) (layer "B.Cu") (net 3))
 (segment (start 112.0775 71.12) (end 112.0775 79.7225) (width 0.2) (layer "B.Cu") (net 3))
 (segment (start 112.0775 52.07) (end 121.6025 42.545) (width 0.2) (layer "B.Cu") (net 3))
 (segment (start 88.55625 86.2) (end 85.7 83.34375) (width 0.2) (layer "B.Cu") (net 3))
 (segment (start 112.0775 79.7225) (end 105.6 86.2) (width 0.2) (layer "B.Cu") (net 3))
 (segment (start 105.6 86.2) (end 88.55625 86.2) (width 0.2) (layer "B.Cu") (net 3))
 (segment (start 131.1275 71.12) (end 131.1275 52.07) (width 0.2) (layer "B.Cu") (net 11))
 (segment (start 131.1275 41.737684) (end 139.845184 33.02) (width 0.2) (layer "B.Cu") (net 11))
 (segment (start 124.4 87.6) (end 87.41625 87.6) (width 0.2) (layer "B.Cu") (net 11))
 (segment (start 131.1275 71.12) (end 131.1275 80.8725) (width 0.2) (layer "B.Cu") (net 11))
 (segment (start 139.845184 33.02) (end 140.63 33.02) (width 0.2) (layer "B.Cu") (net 11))
 (segment (start 87.41625 87.6) (end 83.16 83.34375) (width 0.2) (layer "B.Cu") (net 11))
 (segment (start 131.1275 52.07) (end 131.1275 41.737684) (width 0.2) (layer "B.Cu") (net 11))
 (segment (start 131.1275 80.8725) (end 124.4 87.6) (width 0.2) (layer "B.Cu") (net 11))
 (segment (start 85.87625 88.6) (end 80.62 83.34375) (width 0.2) (layer "B.Cu") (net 8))
 (segment (start 93.19275 48.49275) (end 96.4 51.7) (width 0.2) (layer "B.Cu") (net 8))
 (segment (start 96.4 79.4) (end 95.8 80) (width 0.2) (layer "B.Cu") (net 8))
 (segment (start 95.8 80) (end 83.96375 80) (width 0.2) (layer "B.Cu") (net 8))
 (segment (start 82.40625 49.79375) (end 83.70725 48.49275) (width 0.2) (layer "B.Cu") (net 8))
 (segment (start 143.3 88.6) (end 85.87625 88.6) (width 0.2) (layer "B.Cu") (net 8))
 (segment (start 150.1775 81.7225) (end 143.3 88.6) (width 0.2) (layer "B.Cu") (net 8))
 (segment (start 83.96375 80) (end 80.62 83.34375) (width 0.2) (layer "B.Cu") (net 8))
 (segment (start 150.1775 71.12) (end 150.1775 52.07) (width 0.2) (layer "B.Cu") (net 8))
 (segment (start 96.4 51.7) (end 96.4 79.4) (width 0.2) (layer "B.Cu") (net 8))
 (segment (start 83.70725 48.49275) (end 93.19275 48.49275) (width 0.2) (layer "B.Cu") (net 8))
 (segment (start 150.1775 71.12) (end 150.1775 81.7225) (width 0.2) (layer "B.Cu") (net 8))
 (segment (start 87.40625 64.29375) (end 87.40625 67.27) (width 0.2) (layer "F.Cu") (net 15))
 (segment (start 87.40625 67.27) (end 88.24 68.10375) (width 0.2) (layer "F.Cu") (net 15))
 (segment (start 79.30625 56.79375) (end 90.50625 56.79375) (width 0.2) (layer "F.Cu") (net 17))
 (segment (start 82.40625 64.29375) (end 82.503626 64.29375) (width 0.2) (layer "F.Cu") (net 14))
 (segment (start 85.7 67.490124) (end 85.7 68.10375) (width 0.2) (layer "F.Cu") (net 14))
 (segment (start 82.503626 64.29375) (end 85.7 67.490124) (width 0.2) (layer "F.Cu") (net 14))
 (segment (start 76.8 62.8) (end 78.08 64.08) (width 0.2) (layer "F.Cu") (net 19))
 (segment (start 76.8 39.7) (end 76.8 62.8) (width 0.2) (layer "F.Cu") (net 19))
 (segment (start 108.2 36.42) (end 80.08 36.42) (width 0.2) (layer "F.Cu") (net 19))
 (segment (start 78.08 64.08) (end 78.08 68.10375) (width 0.2) (layer "F.Cu") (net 19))
 (segment (start 80.08 36.42) (end 76.8 39.7) (width 0.2) (layer "F.Cu") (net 19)))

